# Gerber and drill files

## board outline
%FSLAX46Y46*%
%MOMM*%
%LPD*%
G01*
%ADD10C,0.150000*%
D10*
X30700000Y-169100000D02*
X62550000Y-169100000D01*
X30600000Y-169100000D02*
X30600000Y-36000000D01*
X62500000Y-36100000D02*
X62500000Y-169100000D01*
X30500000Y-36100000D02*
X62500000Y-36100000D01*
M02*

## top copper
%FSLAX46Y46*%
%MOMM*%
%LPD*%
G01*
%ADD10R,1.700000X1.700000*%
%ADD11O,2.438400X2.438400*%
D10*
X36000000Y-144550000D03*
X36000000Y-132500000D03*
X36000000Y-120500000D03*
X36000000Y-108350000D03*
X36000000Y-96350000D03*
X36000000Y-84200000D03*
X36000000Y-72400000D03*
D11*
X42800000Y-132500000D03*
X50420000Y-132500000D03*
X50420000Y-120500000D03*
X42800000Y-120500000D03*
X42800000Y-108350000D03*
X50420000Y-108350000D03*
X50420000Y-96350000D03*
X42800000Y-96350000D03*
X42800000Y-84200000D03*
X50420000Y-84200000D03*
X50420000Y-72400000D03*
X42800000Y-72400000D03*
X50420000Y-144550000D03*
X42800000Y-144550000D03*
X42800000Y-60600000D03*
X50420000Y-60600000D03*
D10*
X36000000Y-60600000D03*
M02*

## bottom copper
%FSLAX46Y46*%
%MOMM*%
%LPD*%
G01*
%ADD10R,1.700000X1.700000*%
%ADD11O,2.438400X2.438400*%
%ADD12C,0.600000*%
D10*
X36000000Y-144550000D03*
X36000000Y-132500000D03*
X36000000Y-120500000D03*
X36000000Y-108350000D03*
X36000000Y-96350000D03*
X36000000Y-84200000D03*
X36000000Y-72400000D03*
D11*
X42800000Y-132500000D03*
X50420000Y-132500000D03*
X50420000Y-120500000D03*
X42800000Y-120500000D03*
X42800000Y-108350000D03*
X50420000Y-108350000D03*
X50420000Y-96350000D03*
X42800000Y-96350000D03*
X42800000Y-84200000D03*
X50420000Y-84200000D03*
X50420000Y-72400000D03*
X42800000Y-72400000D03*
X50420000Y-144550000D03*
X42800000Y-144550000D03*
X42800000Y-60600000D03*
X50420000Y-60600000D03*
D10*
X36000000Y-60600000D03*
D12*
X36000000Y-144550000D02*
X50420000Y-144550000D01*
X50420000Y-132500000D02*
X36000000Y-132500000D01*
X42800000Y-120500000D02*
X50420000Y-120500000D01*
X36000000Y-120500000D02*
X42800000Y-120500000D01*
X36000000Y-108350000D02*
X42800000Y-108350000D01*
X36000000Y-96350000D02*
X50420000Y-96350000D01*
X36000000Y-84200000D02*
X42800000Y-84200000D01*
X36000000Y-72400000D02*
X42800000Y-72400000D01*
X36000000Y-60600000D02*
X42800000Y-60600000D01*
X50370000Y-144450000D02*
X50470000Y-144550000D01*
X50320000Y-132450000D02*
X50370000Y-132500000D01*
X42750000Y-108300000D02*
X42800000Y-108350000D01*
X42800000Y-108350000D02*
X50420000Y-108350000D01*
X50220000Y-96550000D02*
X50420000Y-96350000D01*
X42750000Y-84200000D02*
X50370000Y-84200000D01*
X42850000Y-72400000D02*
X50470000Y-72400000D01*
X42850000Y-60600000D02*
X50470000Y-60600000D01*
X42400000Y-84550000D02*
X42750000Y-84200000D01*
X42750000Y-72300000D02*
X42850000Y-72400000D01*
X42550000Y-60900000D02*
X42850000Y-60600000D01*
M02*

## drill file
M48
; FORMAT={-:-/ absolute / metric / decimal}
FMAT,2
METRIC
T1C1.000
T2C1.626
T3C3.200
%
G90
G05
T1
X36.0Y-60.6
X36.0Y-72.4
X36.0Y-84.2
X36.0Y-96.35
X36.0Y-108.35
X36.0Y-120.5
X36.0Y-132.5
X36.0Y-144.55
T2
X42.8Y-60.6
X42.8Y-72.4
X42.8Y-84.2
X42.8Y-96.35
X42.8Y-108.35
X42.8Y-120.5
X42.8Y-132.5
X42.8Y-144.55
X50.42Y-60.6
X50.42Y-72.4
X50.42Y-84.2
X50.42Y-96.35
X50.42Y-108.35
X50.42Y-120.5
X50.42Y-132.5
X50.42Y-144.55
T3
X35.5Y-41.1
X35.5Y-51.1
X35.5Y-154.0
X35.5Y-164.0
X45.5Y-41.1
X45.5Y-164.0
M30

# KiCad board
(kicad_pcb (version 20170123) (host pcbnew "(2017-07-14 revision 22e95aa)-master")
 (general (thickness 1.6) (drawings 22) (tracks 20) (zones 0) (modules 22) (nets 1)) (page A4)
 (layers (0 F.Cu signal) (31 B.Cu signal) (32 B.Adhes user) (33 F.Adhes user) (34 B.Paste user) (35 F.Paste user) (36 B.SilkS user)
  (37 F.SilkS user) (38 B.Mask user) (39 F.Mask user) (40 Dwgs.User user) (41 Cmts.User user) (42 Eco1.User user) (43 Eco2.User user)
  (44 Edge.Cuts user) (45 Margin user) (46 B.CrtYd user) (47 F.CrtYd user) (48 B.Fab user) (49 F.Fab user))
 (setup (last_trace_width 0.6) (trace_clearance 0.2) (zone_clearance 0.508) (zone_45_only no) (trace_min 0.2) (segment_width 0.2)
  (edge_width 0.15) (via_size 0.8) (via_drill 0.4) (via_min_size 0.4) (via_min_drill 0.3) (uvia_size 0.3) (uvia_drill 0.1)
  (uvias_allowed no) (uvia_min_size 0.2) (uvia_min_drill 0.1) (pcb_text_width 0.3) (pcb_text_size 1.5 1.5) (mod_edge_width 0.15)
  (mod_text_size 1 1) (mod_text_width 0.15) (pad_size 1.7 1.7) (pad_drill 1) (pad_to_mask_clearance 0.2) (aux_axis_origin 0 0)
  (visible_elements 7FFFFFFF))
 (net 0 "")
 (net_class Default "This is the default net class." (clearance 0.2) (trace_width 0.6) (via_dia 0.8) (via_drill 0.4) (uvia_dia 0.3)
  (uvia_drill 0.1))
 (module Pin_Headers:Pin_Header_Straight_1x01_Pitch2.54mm (layer F.Cu) (at 36 144.55)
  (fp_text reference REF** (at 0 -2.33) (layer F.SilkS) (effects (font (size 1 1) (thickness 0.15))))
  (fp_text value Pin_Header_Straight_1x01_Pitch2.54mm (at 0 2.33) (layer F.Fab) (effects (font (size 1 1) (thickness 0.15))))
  (pad 1 thru_hole rect (at 0 0) (size 1.7 1.7) (drill 1) (layers *.Cu *.Mask)))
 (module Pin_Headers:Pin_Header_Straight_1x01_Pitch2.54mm (layer F.Cu) (at 36 132.5)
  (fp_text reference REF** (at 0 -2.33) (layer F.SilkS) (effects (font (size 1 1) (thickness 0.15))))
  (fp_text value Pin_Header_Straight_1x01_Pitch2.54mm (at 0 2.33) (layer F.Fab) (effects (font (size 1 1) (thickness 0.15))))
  (pad 1 thru_hole rect (at 0 0) (size 1.7 1.7) (drill 1) (layers *.Cu *.Mask)))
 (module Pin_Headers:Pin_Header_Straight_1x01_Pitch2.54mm (layer F.Cu) (at 36 120.5)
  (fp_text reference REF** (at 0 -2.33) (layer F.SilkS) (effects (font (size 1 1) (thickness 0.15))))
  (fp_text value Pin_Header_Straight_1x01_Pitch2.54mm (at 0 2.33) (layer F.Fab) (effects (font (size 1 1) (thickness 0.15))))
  (pad 1 thru_hole rect (at 0 0) (size 1.7 1.7) (drill 1) (layers *.Cu *.Mask)))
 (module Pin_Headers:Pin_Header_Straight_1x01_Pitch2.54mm (layer F.Cu) (at 36 108.35)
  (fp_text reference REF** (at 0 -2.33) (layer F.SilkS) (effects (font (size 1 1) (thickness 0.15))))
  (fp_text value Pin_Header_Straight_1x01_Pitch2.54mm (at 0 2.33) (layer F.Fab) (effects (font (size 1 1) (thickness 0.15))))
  (pad 1 thru_hole rect (at 0 0) (size 1.7 1.7) (drill 1) (layers *.Cu *.Mask)))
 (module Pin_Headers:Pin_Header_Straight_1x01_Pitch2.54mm (layer F.Cu) (at 36 96.35)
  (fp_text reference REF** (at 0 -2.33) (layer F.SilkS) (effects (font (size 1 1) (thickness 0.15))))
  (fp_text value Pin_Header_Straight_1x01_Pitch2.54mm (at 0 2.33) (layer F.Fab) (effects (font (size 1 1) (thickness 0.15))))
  (pad 1 thru_hole rect (at 0 0) (size 1.7 1.7) (drill 1) (layers *.Cu *.Mask)))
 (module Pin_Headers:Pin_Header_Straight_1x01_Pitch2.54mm (layer F.Cu) (at 36 84.2)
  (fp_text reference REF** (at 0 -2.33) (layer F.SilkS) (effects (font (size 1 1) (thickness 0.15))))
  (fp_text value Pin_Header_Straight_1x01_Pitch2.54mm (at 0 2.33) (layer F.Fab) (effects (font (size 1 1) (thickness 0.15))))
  (pad 1 thru_hole rect (at 0 0) (size 1.7 1.7) (drill 1) (layers *.Cu *.Mask)))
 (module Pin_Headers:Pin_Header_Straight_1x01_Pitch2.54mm (layer F.Cu) (at 36 72.4)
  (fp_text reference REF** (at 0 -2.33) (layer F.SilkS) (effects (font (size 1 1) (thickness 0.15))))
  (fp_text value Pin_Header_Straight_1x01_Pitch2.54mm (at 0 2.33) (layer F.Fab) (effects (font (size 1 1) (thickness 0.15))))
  (pad 1 thru_hole rect (at 0 0) (size 1.7 1.7) (drill 1) (layers *.Cu *.Mask)))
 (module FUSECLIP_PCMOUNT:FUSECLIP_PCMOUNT (layer F.Cu) (at 42.8 132.5)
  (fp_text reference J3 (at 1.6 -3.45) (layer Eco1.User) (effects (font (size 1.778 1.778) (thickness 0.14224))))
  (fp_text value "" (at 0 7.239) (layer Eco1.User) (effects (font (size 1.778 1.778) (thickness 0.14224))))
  (pad 1 thru_hole oval (at 0 0) (size 2.4384 2.4384) (drill 1.6256) (layers *.Cu *.Mask))
  (pad 2 thru_hole oval (at 7.62 0) (size 2.4384 2.4384) (drill 1.6256) (layers *.Cu *.Mask)))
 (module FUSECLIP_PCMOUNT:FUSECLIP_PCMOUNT (layer F.Cu) (at 42.8 120.5)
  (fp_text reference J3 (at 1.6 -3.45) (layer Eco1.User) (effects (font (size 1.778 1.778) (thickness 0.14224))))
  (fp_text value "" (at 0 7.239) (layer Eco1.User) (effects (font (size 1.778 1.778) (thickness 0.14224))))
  (pad 2 thru_hole oval (at 7.62 0) (size 2.4384 2.4384) (drill 1.6256) (layers *.Cu *.Mask))
  (pad 1 thru_hole oval (at 0 0) (size 2.4384 2.4384) (drill 1.6256) (layers *.Cu *.Mask)))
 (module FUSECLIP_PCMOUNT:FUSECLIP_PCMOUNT (layer F.Cu) (at 42.8 108.35)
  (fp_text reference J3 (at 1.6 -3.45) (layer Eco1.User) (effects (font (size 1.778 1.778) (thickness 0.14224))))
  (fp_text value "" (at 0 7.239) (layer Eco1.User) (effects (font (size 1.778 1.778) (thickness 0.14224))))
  (pad 1 thru_hole oval (at 0 0) (size 2.4384 2.4384) (drill 1.6256) (layers *.Cu *.Mask))
  (pad 2 thru_hole oval (at 7.62 0) (size 2.4384 2.4384) (drill 1.6256) (layers *.Cu *.Mask)))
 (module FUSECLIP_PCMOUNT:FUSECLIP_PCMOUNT (layer F.Cu) (at 42.8 96.35)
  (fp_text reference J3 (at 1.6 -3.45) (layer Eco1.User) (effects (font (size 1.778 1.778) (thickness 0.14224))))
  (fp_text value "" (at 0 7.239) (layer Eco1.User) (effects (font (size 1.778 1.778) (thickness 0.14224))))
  (pad 2 thru_hole oval (at 7.62 0) (size 2.4384 2.4384) (drill 1.6256) (layers *.Cu *.Mask))
  (pad 1 thru_hole oval (at 0 0) (size 2.4384 2.4384) (drill 1.6256) (layers *.Cu *.Mask)))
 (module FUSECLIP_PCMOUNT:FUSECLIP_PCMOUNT (layer F.Cu) (at 42.8 84.2)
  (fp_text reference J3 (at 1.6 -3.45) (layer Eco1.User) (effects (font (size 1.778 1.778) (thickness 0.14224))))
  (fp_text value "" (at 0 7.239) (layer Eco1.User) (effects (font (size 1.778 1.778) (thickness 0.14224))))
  (pad 1 thru_hole oval (at 0 0) (size 2.4384 2.4384) (drill 1.6256) (layers *.Cu *.Mask))
  (pad 2 thru_hole oval (at 7.62 0) (size 2.4384 2.4384) (drill 1.6256) (layers *.Cu *.Mask)))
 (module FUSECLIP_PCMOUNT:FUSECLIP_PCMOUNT (layer F.Cu) (at 42.8 72.4)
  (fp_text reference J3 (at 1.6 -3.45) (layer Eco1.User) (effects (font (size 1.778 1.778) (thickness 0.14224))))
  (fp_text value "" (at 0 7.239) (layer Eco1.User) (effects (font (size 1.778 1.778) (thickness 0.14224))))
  (pad 2 thru_hole oval (at 7.62 0) (size 2.4384 2.4384) (drill 1.6256) (layers *.Cu *.Mask))
  (pad 1 thru_hole oval (at 0 0) (size 2.4384 2.4384) (drill 1.6256) (layers *.Cu *.Mask)))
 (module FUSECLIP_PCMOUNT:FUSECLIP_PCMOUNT (layer F.Cu) (at 42.8 144.55)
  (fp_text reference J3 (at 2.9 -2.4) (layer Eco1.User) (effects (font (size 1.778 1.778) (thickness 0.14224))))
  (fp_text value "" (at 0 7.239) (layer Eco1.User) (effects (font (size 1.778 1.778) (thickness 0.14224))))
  (pad 2 thru_hole oval (at 7.62 0) (size 2.4384 2.4384) (drill 1.6256) (layers *.Cu *.Mask))
  (pad 1 thru_hole oval (at 0 0) (size 2.4384 2.4384) (drill 1.6256) (layers *.Cu *.Mask)))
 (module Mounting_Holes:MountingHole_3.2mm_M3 (layer F.Cu) (at 35.5 154)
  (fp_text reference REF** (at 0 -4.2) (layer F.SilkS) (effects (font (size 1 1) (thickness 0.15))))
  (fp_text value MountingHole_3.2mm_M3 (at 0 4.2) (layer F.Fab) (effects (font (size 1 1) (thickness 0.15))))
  (pad "" np_thru_hole circle (at 0 0) (size 3.2 3.2) (drill 3.2) (layers *.Cu *.Mask)))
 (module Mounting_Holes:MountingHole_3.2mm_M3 (layer F.Cu) (at 35.4 51.1)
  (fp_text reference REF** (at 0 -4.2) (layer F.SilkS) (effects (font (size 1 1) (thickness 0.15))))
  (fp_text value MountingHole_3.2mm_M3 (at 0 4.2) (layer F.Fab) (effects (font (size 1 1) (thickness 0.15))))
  (pad "" np_thru_hole circle (at 0.1 0) (size 3.2 3.2) (drill 3.2) (layers *.Cu *.Mask)))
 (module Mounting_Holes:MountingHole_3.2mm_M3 (layer F.Cu) (at 45.5 164)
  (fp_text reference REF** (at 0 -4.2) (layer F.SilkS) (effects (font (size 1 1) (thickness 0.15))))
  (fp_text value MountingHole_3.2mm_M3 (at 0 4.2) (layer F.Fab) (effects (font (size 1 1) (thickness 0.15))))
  (pad "" np_thru_hole circle (at 0 0) (size 3.2 3.2) (drill 3.2) (layers *.Cu *.Mask)))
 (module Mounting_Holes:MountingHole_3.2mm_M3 (layer F.Cu) (at 35.5 41.1)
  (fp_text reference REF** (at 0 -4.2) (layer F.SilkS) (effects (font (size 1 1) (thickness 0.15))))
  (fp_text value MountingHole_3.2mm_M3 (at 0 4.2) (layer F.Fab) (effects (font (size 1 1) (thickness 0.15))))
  (pad 1 np_thru_hole circle (at 0 0) (size 3.2 3.2) (drill 3.2) (layers *.Cu *.Mask)))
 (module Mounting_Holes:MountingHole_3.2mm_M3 (layer F.Cu) (at 35.65 164)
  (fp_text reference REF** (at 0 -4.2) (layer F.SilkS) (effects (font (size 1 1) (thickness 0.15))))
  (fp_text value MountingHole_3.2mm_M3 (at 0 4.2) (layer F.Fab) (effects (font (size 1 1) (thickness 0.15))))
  (pad "" np_thru_hole circle (at -0.15 0) (size 3.2 3.2) (drill 3.2) (layers *.Cu *.Mask)))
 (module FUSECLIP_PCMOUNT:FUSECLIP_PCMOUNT (layer F.Cu) (at 42.8 60.6)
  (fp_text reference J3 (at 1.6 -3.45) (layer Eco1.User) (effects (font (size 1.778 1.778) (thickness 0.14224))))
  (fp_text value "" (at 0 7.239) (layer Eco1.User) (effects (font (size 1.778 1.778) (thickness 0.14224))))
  (pad 1 thru_hole oval (at 0 0) (size 2.4384 2.4384) (drill 1.6256) (layers *.Cu *.Mask))
  (pad 2 thru_hole oval (at 7.62 0) (size 2.4384 2.4384) (drill 1.6256) (layers *.Cu *.Mask)))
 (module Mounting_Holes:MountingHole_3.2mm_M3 (layer F.Cu) (at 45.5 41.2)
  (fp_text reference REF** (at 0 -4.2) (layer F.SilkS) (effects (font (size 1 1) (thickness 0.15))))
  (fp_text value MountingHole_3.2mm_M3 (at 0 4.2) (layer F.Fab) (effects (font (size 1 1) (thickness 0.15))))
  (pad "" np_thru_hole circle (at 0 -0.1) (size 3.2 3.2) (drill 3.2) (layers *.Cu *.Mask)))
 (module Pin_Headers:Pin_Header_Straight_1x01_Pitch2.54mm (layer F.Cu) (at 35.9 60.6)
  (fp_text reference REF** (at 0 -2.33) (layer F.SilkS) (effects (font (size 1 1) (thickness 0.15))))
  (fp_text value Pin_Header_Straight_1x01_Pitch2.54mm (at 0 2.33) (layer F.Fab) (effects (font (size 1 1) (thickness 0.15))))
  (pad 1 thru_hole rect (at 0.1 0) (size 1.7 1.7) (drill 1) (layers *.Cu *.Mask)))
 (gr_line (start 30.7 169.1) (end 62.55 169.1) (angle 90) (layer Edge.Cuts) (width 0.15))
 (gr_line (start 30.6 169.1) (end 30.6 36) (angle 90) (layer Edge.Cuts) (width 0.15))
 (gr_line (start 62.5 36.1) (end 62.5 169.1) (angle 90) (layer Edge.Cuts) (width 0.15))
 (gr_line (start 30.5 36.1) (end 62.5 36.1) (angle 90) (layer Edge.Cuts) (width 0.15))
 (segment (start 36 144.55) (end 50.42 144.55) (width 0.6) (layer B.Cu) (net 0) (status C00000))
 (segment (start 50.42 132.5) (end 36 132.5) (width 0.6) (layer B.Cu) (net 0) (status C00000))
 (segment (start 42.8 120.5) (end 50.42 120.5) (width 0.6) (layer B.Cu) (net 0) (status C00000))
 (segment (start 36 120.5) (end 42.8 120.5) (width 0.6) (layer B.Cu) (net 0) (status C00000))
 (segment (start 36 108.35) (end 42.8 108.35) (width 0.6) (layer B.Cu) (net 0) (status C00000))
 (segment (start 36 96.35) (end 50.42 96.35) (width 0.6) (layer B.Cu) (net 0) (status C00000))
 (segment (start 36 84.2) (end 42.8 84.2) (width 0.6) (layer B.Cu) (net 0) (status C00000))
 (segment (start 36 72.4) (end 42.8 72.4) (width 0.6) (layer B.Cu) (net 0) (status C00000))
 (segment (start 36 60.6) (end 42.8 60.6) (width 0.6) (layer B.Cu) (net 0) (status C00000))
 (segment (start 50.37 144.45) (end 50.47 144.55) (width 0.6) (layer B.Cu) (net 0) (status C00000))
 (segment (start 50.32 132.45) (end 50.37 132.5) (width 0.6) (layer B.Cu) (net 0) (status C00000))
 (segment (start 42.75 108.3) (end 42.8 108.35) (width 0.6) (layer B.Cu) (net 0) (status C00000))
 (segment (start 42.8 108.35) (end 50.42 108.35) (width 0.6) (layer B.Cu) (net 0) (status C00000))
 (segment (start 50.22 96.55) (end 50.42 96.35) (width 0.6) (layer B.Cu) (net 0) (status C00000))
 (segment (start 42.75 84.2) (end 50.37 84.2) (width 0.6) (layer B.Cu) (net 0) (status C00000))
 (segment (start 42.85 72.4) (end 50.47 72.4) (width 0.6) (layer B.Cu) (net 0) (status C00000))
 (segment (start 42.85 60.6) (end 50.47 60.6) (width 0.6) (layer B.Cu) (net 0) (status C00000))
 (segment (start 42.4 84.55) (end 42.75 84.2) (width 0.6) (layer B.Cu) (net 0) (status C00000))
 (segment (start 42.75 72.3) (end 42.85 72.4) (width 0.6) (layer B.Cu) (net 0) (status C00000))
 (segment (start 42.55 60.9) (end 42.85 60.6) (width 0.6) (layer B.Cu) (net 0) (status C00000)))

